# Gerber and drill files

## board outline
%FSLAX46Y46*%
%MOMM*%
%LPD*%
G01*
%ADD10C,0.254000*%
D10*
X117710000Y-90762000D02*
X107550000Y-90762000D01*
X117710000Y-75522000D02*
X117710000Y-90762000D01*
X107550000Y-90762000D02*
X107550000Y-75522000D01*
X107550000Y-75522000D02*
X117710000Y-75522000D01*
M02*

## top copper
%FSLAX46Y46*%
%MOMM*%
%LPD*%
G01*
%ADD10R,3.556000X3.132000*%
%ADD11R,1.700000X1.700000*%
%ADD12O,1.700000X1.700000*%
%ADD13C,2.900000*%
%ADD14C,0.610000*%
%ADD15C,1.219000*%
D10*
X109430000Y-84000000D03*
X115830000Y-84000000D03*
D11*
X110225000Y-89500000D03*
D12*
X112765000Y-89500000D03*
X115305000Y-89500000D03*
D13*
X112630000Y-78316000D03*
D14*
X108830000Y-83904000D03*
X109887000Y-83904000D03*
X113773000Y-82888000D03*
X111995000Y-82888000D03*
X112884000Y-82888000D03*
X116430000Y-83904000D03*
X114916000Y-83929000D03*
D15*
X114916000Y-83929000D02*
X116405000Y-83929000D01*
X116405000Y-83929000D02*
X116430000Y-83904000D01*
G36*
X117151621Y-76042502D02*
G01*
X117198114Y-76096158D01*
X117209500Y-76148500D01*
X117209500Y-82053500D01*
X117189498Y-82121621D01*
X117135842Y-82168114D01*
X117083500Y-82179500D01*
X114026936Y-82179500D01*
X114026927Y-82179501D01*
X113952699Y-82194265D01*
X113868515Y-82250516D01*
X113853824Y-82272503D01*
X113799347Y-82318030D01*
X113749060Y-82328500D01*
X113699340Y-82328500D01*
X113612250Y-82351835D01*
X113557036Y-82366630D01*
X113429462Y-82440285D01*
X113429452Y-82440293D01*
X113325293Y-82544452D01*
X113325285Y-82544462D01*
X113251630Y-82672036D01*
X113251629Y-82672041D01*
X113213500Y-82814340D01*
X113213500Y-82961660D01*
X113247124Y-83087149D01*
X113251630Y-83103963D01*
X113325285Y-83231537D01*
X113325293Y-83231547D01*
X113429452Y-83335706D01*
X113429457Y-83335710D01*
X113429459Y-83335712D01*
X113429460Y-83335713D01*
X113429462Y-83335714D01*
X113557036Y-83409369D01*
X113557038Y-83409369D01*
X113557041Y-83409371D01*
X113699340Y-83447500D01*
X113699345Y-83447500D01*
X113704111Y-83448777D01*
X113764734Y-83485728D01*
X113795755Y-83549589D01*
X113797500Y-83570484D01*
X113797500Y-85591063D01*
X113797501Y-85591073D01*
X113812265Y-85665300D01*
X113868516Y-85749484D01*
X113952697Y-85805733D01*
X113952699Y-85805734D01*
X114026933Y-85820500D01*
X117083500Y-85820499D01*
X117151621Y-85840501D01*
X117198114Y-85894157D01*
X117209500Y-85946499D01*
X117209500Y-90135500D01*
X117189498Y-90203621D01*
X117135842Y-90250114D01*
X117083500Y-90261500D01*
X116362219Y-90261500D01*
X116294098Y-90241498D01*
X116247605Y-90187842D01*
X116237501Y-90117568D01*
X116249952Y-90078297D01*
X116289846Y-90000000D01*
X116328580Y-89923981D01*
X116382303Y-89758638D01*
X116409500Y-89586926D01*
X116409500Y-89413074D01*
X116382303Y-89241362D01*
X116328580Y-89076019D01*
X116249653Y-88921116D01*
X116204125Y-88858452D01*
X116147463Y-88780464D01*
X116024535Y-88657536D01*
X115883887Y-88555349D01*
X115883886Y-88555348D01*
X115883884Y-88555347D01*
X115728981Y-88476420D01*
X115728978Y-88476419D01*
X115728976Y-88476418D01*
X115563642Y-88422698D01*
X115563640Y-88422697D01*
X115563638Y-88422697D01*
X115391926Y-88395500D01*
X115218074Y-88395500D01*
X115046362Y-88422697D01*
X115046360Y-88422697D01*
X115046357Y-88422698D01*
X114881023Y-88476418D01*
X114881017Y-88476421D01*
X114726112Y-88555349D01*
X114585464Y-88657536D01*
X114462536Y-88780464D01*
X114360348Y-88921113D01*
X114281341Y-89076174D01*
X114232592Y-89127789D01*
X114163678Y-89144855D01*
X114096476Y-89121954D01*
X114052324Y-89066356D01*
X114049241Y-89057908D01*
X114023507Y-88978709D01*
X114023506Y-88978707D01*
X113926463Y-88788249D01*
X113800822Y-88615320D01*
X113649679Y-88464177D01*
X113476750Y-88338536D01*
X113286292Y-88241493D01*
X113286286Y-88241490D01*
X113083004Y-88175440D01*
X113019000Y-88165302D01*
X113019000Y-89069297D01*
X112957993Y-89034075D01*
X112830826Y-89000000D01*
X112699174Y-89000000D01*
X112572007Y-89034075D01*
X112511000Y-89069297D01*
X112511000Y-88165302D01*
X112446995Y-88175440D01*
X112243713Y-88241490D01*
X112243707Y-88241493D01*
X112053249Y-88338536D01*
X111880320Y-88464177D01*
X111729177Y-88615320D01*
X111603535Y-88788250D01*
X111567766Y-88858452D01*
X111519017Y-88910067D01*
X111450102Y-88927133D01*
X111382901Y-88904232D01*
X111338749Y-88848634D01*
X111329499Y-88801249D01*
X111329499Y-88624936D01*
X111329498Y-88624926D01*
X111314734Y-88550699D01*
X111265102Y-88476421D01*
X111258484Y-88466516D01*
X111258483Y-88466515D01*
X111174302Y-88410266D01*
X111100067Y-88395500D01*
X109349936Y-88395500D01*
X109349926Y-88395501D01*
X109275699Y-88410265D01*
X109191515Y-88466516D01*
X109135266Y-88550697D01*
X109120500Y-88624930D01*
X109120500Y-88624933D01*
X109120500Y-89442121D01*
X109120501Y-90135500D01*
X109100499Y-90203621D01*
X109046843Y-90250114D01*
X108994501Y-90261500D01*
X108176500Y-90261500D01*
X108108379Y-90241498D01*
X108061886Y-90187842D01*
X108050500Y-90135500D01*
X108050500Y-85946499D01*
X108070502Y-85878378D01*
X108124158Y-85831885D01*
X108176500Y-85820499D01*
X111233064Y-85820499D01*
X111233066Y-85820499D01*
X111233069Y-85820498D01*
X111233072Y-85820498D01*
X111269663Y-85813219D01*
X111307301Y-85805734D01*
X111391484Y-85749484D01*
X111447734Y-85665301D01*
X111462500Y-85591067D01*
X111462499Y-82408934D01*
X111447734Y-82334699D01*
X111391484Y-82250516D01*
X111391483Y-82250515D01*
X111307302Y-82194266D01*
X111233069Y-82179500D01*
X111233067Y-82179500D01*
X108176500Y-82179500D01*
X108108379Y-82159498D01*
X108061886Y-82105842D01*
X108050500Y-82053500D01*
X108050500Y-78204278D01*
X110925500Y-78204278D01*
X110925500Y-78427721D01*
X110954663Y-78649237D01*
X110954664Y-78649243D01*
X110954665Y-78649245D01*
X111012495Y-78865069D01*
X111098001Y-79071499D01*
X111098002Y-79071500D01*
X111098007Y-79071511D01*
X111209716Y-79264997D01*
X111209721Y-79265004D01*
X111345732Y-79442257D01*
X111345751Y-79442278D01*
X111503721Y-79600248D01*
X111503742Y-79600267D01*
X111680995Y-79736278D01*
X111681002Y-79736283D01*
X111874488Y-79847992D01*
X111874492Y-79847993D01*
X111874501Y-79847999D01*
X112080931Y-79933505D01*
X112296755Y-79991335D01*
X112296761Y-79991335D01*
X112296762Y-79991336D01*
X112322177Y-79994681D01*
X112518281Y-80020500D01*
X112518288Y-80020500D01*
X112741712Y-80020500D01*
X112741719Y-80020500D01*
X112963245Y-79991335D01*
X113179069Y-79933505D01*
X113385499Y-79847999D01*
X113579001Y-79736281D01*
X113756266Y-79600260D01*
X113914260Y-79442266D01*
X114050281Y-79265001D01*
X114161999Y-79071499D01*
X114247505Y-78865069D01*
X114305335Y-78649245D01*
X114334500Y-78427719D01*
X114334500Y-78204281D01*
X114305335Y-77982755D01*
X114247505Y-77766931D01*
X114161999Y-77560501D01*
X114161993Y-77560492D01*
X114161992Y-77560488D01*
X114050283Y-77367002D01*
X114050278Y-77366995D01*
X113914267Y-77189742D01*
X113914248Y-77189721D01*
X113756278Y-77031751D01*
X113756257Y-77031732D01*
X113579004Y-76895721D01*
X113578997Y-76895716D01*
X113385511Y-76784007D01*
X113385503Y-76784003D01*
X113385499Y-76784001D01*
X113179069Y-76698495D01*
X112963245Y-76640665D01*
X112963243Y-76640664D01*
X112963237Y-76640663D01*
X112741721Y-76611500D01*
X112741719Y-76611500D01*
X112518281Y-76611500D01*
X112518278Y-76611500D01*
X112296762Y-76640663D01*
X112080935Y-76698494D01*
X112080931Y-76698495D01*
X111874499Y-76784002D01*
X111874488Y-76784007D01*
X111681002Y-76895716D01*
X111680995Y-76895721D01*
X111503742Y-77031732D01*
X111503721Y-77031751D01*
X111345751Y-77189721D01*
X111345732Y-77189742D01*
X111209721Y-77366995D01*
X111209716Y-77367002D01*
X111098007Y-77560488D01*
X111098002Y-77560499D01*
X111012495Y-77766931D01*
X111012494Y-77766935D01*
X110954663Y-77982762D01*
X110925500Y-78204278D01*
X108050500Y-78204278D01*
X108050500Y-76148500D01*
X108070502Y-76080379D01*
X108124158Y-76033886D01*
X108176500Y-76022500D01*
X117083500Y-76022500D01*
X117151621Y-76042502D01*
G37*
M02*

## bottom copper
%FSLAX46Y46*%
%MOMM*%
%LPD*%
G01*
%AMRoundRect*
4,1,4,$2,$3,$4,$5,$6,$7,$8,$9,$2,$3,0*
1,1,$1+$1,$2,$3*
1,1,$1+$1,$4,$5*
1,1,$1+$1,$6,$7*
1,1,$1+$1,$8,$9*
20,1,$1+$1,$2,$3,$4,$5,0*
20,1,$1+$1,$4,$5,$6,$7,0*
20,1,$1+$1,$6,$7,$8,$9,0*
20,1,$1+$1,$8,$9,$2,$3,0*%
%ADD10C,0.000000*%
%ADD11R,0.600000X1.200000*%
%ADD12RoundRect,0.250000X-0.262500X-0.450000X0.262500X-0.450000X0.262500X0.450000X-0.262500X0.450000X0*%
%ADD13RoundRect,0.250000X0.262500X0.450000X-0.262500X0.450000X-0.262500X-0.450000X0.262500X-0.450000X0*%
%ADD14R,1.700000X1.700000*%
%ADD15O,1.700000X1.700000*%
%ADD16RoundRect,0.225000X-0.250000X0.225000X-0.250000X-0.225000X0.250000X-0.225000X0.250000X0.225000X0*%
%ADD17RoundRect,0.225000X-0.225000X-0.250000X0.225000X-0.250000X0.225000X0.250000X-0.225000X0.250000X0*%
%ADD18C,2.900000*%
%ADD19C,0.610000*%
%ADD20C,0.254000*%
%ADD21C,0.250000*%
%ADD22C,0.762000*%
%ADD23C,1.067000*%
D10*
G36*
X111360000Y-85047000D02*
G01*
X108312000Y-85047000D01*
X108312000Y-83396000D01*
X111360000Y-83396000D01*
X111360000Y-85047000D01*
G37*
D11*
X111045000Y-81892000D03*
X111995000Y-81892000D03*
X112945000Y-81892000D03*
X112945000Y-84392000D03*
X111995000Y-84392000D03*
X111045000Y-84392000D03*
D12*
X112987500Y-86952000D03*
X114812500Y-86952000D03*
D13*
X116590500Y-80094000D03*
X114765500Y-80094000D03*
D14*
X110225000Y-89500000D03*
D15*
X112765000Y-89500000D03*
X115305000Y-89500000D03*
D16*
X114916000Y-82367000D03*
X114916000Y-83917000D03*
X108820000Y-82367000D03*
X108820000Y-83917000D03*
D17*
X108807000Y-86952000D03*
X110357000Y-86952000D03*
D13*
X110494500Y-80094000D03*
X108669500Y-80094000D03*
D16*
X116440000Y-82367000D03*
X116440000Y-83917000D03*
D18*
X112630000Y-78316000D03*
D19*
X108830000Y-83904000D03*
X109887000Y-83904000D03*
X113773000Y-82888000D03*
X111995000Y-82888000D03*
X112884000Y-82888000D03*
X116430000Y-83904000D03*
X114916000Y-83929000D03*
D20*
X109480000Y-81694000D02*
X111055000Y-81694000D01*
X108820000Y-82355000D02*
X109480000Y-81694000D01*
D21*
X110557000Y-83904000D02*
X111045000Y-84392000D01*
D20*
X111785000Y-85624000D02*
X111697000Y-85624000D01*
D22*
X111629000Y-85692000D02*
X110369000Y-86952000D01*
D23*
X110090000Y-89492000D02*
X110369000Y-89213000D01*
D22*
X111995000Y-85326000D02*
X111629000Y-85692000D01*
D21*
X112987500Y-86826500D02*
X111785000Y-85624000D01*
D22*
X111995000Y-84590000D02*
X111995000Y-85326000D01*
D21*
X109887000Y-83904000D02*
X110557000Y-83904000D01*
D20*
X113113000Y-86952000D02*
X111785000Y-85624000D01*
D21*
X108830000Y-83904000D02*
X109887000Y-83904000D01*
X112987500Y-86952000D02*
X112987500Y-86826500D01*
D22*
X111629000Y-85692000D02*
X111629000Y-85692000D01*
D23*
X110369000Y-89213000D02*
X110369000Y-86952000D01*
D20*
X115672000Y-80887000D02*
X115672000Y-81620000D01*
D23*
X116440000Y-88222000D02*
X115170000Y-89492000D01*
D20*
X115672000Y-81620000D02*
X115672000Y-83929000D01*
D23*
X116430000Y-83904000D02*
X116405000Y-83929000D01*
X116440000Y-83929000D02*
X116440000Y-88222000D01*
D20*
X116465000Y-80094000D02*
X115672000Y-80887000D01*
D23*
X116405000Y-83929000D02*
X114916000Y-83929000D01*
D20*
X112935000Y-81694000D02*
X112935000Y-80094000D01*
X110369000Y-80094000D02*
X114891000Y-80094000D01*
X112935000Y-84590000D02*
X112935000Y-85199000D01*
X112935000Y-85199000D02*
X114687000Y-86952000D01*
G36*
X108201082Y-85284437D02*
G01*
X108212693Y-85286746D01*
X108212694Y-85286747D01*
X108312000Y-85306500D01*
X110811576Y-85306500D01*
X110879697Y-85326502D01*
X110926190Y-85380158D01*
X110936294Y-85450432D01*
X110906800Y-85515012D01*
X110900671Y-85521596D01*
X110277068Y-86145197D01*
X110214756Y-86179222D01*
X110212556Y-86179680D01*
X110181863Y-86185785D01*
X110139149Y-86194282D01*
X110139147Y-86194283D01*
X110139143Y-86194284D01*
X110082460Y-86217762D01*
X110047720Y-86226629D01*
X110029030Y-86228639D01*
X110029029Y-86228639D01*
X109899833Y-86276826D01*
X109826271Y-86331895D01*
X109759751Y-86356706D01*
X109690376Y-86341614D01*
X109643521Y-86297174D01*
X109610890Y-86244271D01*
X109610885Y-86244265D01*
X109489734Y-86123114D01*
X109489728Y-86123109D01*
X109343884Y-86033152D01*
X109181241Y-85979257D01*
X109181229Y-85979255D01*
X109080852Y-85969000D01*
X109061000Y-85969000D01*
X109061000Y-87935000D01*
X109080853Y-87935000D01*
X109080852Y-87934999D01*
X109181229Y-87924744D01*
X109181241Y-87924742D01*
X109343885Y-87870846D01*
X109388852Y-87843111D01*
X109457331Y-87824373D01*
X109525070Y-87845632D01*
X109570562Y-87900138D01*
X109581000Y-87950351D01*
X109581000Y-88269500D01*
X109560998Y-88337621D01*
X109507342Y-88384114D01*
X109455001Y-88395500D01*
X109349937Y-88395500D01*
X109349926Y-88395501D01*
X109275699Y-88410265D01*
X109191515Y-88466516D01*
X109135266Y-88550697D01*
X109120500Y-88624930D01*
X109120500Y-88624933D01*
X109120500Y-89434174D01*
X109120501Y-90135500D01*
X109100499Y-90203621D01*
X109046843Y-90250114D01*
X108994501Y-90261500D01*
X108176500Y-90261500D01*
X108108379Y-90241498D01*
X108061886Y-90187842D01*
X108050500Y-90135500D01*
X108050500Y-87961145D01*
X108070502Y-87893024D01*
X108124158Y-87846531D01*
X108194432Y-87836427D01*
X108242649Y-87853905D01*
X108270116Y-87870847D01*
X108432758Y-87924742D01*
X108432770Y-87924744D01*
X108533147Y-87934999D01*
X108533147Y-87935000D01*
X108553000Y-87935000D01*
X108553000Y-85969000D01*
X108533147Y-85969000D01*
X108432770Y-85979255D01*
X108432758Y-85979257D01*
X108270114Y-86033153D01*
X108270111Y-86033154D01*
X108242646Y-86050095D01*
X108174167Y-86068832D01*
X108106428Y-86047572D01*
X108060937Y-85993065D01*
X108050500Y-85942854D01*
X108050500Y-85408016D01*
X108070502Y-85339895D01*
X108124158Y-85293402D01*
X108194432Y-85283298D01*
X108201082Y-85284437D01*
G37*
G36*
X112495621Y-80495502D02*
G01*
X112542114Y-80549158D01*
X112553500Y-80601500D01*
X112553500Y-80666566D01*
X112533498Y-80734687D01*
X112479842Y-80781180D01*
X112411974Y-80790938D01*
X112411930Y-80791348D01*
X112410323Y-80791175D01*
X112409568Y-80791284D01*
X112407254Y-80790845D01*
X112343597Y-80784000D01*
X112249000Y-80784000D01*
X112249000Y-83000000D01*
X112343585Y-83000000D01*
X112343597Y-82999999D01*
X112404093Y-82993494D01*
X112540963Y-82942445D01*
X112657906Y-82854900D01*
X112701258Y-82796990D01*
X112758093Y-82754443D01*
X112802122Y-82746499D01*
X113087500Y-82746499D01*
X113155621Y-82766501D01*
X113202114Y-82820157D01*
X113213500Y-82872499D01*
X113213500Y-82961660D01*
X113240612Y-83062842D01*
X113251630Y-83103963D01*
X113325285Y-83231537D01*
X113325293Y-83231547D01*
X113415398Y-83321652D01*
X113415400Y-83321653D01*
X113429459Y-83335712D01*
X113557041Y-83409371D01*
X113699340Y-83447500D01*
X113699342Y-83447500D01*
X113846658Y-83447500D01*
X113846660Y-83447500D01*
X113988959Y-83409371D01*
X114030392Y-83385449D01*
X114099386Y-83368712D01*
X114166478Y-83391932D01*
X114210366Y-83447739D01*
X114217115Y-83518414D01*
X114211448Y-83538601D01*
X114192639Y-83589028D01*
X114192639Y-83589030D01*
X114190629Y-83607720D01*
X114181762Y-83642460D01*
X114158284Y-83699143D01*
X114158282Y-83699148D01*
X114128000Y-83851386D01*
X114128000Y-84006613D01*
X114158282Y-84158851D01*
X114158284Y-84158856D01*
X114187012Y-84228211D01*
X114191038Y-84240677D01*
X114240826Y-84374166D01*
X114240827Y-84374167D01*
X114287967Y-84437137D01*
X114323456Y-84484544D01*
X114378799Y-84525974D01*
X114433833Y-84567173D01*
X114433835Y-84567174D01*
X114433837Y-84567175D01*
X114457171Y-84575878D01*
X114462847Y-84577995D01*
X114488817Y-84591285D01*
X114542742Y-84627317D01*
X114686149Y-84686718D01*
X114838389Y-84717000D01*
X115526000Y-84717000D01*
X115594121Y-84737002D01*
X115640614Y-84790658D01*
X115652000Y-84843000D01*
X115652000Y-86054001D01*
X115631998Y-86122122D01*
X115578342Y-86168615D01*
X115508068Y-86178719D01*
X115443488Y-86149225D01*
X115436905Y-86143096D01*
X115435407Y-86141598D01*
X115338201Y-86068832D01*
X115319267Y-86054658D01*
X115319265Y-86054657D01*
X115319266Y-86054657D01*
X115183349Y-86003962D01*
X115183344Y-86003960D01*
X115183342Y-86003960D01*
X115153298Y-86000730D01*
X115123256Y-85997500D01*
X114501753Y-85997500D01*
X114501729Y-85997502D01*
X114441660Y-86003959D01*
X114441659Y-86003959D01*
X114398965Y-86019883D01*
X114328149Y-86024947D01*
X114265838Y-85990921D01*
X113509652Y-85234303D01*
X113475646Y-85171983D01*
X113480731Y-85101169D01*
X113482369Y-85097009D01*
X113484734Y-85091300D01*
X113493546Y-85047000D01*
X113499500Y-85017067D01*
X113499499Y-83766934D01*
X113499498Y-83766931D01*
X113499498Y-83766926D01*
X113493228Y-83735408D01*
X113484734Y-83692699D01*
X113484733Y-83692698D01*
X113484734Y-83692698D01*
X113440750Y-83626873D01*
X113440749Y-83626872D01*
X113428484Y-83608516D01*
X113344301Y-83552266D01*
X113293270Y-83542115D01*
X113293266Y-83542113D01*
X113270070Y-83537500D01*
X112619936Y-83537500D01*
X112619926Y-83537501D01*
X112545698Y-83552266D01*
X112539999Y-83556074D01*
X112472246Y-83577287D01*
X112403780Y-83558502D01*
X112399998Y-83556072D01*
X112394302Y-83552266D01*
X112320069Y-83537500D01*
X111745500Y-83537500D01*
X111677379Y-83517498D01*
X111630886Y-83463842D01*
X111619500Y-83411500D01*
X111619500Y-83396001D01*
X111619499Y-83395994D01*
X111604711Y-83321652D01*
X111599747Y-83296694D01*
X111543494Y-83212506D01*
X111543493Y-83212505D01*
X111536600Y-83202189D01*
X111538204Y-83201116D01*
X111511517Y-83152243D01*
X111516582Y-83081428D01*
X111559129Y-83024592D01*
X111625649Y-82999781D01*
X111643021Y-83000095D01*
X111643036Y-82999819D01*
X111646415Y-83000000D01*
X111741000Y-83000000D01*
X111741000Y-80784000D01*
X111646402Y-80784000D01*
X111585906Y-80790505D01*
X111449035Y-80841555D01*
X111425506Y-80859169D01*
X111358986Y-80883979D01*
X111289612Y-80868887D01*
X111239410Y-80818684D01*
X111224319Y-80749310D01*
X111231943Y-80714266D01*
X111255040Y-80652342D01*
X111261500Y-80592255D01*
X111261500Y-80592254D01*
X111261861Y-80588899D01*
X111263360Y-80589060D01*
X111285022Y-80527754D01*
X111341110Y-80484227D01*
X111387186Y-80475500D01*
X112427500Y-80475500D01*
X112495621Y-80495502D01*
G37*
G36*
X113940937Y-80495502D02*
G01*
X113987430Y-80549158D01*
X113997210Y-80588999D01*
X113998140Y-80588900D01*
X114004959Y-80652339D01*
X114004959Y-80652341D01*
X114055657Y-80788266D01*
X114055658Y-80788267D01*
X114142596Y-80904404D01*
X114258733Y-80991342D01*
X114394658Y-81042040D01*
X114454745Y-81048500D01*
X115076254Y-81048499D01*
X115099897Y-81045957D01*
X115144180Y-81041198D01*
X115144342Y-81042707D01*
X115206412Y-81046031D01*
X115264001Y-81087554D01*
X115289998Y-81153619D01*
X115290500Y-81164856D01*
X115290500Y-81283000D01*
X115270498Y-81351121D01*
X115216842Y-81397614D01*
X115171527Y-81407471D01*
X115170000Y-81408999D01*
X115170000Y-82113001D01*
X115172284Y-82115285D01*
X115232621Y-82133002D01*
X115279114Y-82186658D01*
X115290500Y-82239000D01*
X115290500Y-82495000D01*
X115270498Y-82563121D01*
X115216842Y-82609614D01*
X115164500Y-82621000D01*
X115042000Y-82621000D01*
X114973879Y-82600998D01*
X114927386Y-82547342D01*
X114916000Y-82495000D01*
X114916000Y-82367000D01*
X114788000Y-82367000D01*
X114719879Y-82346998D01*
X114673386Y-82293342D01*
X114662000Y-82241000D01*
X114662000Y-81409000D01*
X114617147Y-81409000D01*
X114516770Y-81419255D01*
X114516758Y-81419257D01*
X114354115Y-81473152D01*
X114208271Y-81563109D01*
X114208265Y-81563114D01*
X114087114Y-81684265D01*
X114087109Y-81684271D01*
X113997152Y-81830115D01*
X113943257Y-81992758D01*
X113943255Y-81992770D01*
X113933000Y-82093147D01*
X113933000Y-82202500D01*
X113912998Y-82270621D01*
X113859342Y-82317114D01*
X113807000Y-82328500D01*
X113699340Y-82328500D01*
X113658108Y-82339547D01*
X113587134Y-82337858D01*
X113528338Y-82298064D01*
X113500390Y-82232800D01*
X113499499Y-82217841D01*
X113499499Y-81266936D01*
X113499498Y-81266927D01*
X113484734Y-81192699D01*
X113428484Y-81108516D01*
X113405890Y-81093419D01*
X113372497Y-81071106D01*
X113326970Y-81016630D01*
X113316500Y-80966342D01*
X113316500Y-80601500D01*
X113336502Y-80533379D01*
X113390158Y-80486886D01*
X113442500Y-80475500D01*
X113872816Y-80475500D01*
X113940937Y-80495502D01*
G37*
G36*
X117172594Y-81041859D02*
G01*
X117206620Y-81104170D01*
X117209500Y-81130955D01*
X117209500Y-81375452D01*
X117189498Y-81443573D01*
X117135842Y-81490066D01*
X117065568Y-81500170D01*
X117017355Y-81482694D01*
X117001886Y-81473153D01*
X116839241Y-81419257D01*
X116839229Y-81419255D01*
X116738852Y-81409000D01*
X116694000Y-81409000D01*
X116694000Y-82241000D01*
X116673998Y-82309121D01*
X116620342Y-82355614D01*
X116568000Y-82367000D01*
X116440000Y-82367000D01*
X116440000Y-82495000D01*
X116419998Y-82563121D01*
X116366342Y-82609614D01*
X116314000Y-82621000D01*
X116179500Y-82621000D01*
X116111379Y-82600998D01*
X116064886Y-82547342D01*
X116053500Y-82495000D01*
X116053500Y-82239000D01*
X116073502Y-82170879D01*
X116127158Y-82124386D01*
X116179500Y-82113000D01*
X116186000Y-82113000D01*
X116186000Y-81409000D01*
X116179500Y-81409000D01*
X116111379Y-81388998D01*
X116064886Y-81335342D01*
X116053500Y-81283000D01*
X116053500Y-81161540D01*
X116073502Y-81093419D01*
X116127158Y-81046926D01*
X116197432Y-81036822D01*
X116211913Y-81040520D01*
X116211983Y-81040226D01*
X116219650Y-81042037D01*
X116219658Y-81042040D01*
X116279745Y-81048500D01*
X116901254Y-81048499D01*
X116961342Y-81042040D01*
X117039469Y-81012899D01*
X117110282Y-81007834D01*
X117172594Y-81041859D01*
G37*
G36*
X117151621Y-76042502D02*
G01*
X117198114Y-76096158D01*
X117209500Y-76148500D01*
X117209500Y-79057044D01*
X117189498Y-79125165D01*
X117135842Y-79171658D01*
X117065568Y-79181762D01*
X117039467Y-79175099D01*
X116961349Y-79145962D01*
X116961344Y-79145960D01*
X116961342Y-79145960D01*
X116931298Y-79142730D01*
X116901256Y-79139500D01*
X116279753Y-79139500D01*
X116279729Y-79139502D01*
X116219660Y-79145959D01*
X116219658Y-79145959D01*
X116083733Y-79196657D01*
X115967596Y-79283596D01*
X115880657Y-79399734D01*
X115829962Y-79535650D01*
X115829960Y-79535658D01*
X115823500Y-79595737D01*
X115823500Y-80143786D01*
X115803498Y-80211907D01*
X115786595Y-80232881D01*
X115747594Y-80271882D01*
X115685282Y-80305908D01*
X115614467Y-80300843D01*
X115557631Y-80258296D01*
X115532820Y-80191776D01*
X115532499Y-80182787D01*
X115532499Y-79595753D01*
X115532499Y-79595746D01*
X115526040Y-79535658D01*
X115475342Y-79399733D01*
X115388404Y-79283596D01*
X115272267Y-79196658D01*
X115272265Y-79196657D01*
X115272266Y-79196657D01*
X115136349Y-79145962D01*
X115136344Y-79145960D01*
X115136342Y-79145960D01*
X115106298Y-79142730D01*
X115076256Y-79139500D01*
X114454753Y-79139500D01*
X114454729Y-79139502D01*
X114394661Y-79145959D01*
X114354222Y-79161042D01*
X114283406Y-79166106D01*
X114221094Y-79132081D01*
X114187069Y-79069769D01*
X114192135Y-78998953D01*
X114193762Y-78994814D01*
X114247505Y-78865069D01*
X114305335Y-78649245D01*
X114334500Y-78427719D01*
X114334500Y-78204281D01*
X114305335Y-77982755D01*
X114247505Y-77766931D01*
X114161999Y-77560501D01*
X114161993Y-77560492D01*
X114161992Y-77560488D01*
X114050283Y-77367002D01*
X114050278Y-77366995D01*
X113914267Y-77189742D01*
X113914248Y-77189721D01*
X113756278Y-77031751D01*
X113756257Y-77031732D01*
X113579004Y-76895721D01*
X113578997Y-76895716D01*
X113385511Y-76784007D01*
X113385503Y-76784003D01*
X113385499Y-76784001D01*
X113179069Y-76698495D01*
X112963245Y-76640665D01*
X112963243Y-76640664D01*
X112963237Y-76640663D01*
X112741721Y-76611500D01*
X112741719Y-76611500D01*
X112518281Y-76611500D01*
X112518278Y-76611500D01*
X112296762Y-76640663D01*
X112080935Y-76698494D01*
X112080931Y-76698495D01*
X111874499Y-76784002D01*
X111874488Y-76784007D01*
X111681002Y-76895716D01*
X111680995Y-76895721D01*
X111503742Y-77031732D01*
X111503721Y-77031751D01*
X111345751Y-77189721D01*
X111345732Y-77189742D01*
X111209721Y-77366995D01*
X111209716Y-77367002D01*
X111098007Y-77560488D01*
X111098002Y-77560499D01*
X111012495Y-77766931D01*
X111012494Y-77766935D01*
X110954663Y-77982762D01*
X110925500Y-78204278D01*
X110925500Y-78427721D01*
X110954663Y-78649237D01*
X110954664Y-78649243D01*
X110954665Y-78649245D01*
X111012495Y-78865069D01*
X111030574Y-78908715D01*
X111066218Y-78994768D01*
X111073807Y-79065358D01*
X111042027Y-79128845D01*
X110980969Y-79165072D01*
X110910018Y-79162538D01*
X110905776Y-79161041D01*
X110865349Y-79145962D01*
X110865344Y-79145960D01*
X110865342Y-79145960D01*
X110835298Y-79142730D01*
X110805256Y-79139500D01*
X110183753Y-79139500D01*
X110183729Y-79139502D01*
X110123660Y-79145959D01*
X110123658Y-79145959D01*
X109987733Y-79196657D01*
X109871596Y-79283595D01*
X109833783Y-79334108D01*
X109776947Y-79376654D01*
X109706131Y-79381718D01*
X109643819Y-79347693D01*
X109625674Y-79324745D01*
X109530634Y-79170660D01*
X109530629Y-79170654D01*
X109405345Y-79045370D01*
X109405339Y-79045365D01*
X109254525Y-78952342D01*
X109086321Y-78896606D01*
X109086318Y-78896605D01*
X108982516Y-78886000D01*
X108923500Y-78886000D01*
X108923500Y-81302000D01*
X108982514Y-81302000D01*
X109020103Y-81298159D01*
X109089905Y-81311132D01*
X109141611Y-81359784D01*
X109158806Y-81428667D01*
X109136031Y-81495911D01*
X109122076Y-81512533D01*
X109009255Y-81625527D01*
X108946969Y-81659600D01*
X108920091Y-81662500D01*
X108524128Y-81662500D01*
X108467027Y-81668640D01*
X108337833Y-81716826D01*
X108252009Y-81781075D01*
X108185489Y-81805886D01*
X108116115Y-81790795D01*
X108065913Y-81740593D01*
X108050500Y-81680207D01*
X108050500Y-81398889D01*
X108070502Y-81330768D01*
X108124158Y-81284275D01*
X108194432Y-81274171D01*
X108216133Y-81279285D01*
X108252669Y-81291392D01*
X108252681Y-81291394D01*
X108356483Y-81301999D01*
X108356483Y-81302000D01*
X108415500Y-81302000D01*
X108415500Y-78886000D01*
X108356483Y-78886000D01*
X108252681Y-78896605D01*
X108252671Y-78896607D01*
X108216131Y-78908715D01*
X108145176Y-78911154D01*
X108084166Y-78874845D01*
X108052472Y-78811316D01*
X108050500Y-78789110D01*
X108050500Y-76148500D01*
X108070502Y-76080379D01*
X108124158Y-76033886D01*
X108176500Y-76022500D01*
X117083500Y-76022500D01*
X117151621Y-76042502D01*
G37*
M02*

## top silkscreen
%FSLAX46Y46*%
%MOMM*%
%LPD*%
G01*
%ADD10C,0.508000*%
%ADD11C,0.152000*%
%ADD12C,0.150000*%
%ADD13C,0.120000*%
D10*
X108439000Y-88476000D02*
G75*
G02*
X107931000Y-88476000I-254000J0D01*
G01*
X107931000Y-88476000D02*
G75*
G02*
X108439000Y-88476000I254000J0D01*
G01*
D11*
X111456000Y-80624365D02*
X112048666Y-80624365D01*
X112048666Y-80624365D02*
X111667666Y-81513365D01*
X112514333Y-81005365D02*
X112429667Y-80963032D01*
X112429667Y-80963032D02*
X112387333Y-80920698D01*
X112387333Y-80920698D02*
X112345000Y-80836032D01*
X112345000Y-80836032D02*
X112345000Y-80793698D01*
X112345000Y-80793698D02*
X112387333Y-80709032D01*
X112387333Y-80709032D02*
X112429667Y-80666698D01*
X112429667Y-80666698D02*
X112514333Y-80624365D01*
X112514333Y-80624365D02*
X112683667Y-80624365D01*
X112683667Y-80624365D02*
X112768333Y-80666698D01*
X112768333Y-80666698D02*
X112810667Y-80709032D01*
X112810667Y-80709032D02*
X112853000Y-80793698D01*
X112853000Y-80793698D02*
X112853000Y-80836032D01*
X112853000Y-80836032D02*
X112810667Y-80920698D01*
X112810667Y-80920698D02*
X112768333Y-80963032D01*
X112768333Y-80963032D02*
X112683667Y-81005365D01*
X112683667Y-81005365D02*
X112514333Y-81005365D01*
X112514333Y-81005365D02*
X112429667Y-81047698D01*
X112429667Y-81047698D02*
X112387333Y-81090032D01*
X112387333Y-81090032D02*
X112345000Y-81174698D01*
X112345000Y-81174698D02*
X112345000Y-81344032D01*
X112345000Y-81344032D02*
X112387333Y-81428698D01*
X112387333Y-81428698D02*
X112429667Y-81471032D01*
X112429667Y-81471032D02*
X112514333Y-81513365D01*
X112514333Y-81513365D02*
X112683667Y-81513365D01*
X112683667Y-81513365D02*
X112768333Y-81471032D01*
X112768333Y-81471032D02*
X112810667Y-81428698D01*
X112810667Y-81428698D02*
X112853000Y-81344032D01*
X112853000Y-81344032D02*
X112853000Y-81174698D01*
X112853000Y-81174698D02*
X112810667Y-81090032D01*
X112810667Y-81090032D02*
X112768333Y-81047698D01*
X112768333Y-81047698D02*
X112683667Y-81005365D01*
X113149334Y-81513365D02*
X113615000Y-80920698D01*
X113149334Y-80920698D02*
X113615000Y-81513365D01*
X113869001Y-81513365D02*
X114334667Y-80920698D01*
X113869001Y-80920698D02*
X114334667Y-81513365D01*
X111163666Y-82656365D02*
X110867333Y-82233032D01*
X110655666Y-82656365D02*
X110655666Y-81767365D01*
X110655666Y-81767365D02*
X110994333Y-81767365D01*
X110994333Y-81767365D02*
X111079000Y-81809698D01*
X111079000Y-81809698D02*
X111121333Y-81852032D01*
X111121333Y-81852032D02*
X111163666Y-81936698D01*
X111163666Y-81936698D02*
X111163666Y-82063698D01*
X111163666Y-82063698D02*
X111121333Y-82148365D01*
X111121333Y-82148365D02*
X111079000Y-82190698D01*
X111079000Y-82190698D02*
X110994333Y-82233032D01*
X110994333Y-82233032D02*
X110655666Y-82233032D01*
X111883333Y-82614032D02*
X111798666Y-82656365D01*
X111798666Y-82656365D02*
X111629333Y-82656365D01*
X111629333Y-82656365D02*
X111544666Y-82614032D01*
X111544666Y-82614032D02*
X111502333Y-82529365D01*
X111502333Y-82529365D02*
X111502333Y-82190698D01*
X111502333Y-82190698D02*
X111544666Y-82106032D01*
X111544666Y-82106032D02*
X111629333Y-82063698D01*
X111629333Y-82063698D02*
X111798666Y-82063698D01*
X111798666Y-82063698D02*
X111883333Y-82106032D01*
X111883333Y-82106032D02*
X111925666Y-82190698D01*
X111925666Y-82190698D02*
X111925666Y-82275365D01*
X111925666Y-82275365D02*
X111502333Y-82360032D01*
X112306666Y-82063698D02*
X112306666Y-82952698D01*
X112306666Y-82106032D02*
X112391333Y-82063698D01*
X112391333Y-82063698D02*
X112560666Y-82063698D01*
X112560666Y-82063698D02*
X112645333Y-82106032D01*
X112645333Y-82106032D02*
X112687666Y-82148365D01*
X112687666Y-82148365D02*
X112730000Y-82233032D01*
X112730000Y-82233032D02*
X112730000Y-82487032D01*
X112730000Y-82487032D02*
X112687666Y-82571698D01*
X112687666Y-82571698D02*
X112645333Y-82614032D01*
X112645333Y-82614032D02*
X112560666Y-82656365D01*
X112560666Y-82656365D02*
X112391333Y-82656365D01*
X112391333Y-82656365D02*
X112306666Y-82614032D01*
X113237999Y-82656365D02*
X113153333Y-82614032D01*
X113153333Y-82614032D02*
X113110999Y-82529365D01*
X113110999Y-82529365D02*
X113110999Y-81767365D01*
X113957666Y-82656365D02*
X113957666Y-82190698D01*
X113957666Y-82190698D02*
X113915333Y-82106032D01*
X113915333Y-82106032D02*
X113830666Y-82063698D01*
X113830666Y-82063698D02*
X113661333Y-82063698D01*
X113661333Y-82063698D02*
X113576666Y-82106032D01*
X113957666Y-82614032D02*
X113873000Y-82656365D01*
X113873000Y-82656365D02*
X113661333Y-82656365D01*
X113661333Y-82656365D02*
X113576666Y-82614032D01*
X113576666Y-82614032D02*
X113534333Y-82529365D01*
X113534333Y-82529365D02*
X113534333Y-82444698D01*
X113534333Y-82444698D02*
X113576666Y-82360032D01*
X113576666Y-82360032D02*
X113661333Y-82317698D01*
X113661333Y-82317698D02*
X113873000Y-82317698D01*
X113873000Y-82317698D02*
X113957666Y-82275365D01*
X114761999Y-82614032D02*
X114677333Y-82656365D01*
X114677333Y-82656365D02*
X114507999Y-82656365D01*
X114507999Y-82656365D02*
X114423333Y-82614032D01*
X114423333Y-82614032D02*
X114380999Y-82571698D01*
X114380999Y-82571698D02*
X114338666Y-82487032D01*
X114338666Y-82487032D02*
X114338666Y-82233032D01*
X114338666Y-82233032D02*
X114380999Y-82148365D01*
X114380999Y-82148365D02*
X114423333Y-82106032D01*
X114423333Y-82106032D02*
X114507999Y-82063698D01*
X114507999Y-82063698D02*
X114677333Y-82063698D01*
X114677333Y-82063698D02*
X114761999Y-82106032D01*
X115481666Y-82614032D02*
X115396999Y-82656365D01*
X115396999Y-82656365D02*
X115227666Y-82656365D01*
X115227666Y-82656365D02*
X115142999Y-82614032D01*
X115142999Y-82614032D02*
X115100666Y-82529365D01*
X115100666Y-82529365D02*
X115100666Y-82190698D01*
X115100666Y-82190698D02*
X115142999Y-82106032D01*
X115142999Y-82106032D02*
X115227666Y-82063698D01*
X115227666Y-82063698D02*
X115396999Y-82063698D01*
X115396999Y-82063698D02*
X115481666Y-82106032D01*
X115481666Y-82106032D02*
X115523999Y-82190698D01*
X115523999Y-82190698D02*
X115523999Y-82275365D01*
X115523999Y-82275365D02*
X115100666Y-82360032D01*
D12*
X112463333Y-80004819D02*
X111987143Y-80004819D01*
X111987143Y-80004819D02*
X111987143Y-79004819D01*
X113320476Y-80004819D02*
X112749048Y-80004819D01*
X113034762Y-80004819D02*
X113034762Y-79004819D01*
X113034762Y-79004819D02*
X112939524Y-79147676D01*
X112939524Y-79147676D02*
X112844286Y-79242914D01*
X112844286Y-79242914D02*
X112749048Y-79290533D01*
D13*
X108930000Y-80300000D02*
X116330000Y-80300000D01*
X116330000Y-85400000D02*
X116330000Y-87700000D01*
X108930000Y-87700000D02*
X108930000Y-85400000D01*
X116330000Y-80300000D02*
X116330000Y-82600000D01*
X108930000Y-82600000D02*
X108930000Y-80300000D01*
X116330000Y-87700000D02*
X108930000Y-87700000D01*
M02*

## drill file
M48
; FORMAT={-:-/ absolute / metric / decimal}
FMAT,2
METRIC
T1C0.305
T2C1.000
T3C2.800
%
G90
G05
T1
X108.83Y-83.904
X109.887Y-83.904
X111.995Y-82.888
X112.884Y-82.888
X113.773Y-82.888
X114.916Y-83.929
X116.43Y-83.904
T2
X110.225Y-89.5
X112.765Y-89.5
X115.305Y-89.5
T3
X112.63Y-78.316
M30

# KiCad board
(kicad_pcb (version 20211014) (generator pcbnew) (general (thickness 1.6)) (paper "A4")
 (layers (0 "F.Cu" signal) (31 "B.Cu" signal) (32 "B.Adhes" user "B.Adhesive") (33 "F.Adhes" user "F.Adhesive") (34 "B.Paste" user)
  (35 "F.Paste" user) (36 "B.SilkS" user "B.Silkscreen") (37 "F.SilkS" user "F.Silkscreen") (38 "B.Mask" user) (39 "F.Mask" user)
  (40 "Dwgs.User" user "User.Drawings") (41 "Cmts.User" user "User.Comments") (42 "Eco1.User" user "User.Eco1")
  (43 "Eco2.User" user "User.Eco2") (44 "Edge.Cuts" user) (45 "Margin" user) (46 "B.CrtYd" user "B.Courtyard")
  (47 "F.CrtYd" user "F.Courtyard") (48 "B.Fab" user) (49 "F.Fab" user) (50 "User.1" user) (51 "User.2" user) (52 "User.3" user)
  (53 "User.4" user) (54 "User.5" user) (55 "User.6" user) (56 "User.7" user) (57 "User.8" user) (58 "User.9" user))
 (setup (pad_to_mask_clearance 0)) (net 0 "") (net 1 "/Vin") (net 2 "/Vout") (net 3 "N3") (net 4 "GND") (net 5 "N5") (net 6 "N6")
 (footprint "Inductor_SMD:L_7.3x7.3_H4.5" (layer "F.Cu") (at 112.63 84)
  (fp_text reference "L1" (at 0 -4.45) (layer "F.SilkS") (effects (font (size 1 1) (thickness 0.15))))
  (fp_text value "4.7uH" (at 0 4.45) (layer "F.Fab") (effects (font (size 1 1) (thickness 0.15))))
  (fp_line (start -3.7 -3.7) (end 3.7 -3.7) (layer "F.SilkS") (width 0.12))
  (fp_line (start 3.7 1.4) (end 3.7 3.7) (layer "F.SilkS") (width 0.12))
  (fp_line (start -3.7 3.7) (end -3.7 1.4) (layer "F.SilkS") (width 0.12))
  (fp_line (start 3.7 -3.7) (end 3.7 -1.4) (layer "F.SilkS") (width 0.12))
  (fp_line (start -3.7 -1.4) (end -3.7 -3.7) (layer "F.SilkS") (width 0.12))
  (fp_line (start 3.7 3.7) (end -3.7 3.7) (layer "F.SilkS") (width 0.12))
  (pad "1" smd rect (at -3.2 0) (size 3.556 3.132) (layers "F.Cu" "F.Paste" "F.Mask") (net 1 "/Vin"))
  (pad "2" smd rect (at 3.2 0) (size 3.556 3.132) (layers "F.Cu" "F.Paste" "F.Mask") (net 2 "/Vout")))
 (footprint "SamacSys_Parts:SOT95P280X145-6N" (layer "B.Cu") (at 111.995 83.142 -90)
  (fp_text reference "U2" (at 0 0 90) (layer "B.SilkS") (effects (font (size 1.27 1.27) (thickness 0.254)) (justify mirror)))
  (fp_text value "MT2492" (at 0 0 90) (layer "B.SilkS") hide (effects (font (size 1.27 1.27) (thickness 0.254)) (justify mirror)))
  (pad "1" smd rect locked (at -1.25 0.95 180) (size 0.6 1.2) (layers "B.Cu" "B.Paste" "B.Mask") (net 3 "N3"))
  (pad "2" smd rect locked (at -1.25 0 180) (size 0.6 1.2) (layers "B.Cu" "B.Paste" "B.Mask") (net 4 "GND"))
  (pad "3" smd rect locked (at -1.25 -0.95 180) (size 0.6 1.2) (layers "B.Cu" "B.Paste" "B.Mask") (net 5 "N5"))
  (pad "4" smd rect locked (at 1.25 -0.95 180) (size 0.6 1.2) (layers "B.Cu" "B.Paste" "B.Mask") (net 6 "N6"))
  (pad "5" smd rect locked (at 1.25 0 180) (size 0.6 1.2) (layers "B.Cu" "B.Paste" "B.Mask") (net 1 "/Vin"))
  (pad "6" smd rect locked (at 1.25 0.95 180) (size 0.6 1.2) (layers "B.Cu" "B.Paste" "B.Mask") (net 1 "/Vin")))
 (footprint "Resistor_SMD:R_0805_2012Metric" (layer "B.Cu") (at 113.9 86.952)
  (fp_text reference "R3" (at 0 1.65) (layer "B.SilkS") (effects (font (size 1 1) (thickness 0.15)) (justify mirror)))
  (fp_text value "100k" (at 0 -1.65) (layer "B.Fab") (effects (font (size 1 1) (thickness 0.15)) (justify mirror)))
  (pad "1" smd roundrect locked (at -0.9125 0) (size 1.025 1.4) (layers "B.Cu" "B.Paste" "B.Mask") (roundrect_rratio 0.243902)
   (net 1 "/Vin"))
  (pad "2" smd roundrect locked (at 0.9125 0) (size 1.025 1.4) (layers "B.Cu" "B.Paste" "B.Mask") (roundrect_rratio 0.243902) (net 6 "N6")))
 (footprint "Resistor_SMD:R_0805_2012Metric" (layer "B.Cu") (at 115.678 80.094 180)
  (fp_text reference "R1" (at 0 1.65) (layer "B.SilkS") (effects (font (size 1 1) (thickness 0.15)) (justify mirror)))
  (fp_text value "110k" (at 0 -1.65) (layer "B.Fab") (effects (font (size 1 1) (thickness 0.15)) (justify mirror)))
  (pad "1" smd roundrect locked (at -0.9125 0 180) (size 1.025 1.4) (layers "B.Cu" "B.Paste" "B.Mask") (roundrect_rratio 0.243902)
   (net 2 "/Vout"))
  (pad "2" smd roundrect locked (at 0.9125 0 180) (size 1.025 1.4) (layers "B.Cu" "B.Paste" "B.Mask") (roundrect_rratio 0.243902)
   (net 5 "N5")))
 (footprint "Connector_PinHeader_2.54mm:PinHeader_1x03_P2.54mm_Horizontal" (layer "B.Cu") (at 110.225 89.5 -90)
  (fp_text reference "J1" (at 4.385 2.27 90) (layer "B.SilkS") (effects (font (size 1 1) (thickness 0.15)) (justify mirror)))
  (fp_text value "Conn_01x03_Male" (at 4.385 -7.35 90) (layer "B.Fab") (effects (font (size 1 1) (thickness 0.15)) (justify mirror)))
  (pad "1" thru_hole rect locked (at 0 0 270) (size 1.7 1.7) (drill 1) (layers *.Cu *.Mask) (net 1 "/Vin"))
  (pad "2" thru_hole oval locked (at 0 -2.54 270) (size 1.7 1.7) (drill 1) (layers *.Cu *.Mask) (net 4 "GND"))
  (pad "3" thru_hole oval locked (at 0 -5.08 270) (size 1.7 1.7) (drill 1) (layers *.Cu *.Mask) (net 2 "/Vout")))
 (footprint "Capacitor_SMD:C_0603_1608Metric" (layer "B.Cu") (at 114.916 83.142 -90)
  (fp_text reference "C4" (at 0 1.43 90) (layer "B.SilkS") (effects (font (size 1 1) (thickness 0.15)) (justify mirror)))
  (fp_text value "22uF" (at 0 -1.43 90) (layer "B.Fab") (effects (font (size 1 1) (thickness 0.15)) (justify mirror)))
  (pad "1" smd roundrect locked (at -0.775 0 270) (size 0.9 0.95) (layers "B.Cu" "B.Paste" "B.Mask") (roundrect_rratio 0.25) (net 4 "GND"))
  (pad "2" smd roundrect locked (at 0.775 0 270) (size 0.9 0.95) (layers "B.Cu" "B.Paste" "B.Mask") (roundrect_rratio 0.25) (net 2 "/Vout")))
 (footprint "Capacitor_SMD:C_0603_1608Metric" (layer "B.Cu") (at 108.82 83.142 -90)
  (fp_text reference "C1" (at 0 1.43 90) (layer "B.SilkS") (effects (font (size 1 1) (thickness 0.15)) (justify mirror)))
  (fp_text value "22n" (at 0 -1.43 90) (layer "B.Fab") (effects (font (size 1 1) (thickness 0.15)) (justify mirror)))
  (pad "1" smd roundrect locked (at -0.775 0 270) (size 0.9 0.95) (layers "B.Cu" "B.Paste" "B.Mask") (roundrect_rratio 0.25) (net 3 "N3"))
  (pad "2" smd roundrect locked (at 0.775 0 270) (size 0.9 0.95) (layers "B.Cu" "B.Paste" "B.Mask") (roundrect_rratio 0.25) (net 1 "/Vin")))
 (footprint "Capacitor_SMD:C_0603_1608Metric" (layer "B.Cu") (at 109.582 86.952)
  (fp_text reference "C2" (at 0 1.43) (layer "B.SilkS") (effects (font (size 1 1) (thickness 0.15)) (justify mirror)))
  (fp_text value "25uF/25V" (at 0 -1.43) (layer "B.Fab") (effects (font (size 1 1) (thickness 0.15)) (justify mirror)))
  (pad "1" smd roundrect locked (at -0.775 0) (size 0.9 0.95) (layers "B.Cu" "B.Paste" "B.Mask") (roundrect_rratio 0.25) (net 4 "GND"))
  (pad "2" smd roundrect locked (at 0.775 0) (size 0.9 0.95) (layers "B.Cu" "B.Paste" "B.Mask") (roundrect_rratio 0.25) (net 1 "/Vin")))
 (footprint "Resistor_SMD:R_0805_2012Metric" (layer "B.Cu") (at 109.582 80.094 180)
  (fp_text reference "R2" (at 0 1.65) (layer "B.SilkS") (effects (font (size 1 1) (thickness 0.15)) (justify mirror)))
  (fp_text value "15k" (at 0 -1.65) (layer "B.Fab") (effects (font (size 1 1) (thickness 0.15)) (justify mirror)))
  (pad "1" smd roundrect locked (at -0.9125 0 180) (size 1.025 1.4) (layers "B.Cu" "B.Paste" "B.Mask") (roundrect_rratio 0.243902)
   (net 5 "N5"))
  (pad "2" smd roundrect locked (at 0.9125 0 180) (size 1.025 1.4) (layers "B.Cu" "B.Paste" "B.Mask") (roundrect_rratio 0.243902)
   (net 4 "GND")))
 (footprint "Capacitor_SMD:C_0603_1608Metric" (layer "B.Cu") (at 116.44 83.142 -90)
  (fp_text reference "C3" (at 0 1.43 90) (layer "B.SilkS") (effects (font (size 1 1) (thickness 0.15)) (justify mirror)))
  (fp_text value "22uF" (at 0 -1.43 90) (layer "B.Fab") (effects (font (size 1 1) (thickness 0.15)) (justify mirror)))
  (pad "1" smd roundrect locked (at -0.775 0 270) (size 0.9 0.95) (layers "B.Cu" "B.Paste" "B.Mask") (roundrect_rratio 0.25) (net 4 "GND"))
  (pad "2" smd roundrect locked (at 0.775 0 270) (size 0.9 0.95) (layers "B.Cu" "B.Paste" "B.Mask") (roundrect_rratio 0.25) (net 2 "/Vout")))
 (gr_poly (pts (xy 108.312 83.396) (xy 111.36 83.396) (xy 111.36 85.047) (xy 108.312 85.047)) (layer "B.Cu") (width 0) (fill solid))
 (gr_circle (center 108.185 88.476) (end 108.439 88.476) (layer "F.SilkS") (width 0.508) (fill none))
 (gr_line (start 117.71 90.762) (end 107.55 90.762) (layer "Edge.Cuts") (width 0.254))
 (gr_line (start 117.71 75.522) (end 117.71 90.762) (layer "Edge.Cuts") (width 0.254))
 (gr_line (start 107.55 90.762) (end 107.55 75.522) (layer "Edge.Cuts") (width 0.254))
 (gr_line (start 107.55 75.522) (end 117.71 75.522) (layer "Edge.Cuts") (width 0.254))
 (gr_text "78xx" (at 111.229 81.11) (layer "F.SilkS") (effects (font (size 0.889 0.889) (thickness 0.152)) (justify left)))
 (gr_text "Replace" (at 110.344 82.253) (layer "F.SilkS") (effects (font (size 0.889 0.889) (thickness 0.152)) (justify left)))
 (via (at 112.63 78.316) (size 2.9) (drill 2.8) (layers "F.Cu" "B.Cu") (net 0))
 (segment (start 109.48 81.694) (end 111.055 81.694) (width 0.254) (layer "B.Cu") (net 3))
 (segment (start 108.82 82.355) (end 109.48 81.694) (width 0.254) (layer "B.Cu") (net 3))
 (via (at 108.83 83.904) (size 0.61) (drill 0.305) (layers "F.Cu" "B.Cu") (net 1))
 (via (at 109.887 83.904) (size 0.61) (drill 0.305) (layers "F.Cu" "B.Cu") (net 1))
 (segment (start 110.557 83.904) (end 111.045 84.392) (width 0.25) (layer "B.Cu") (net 1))
 (segment (start 111.785 85.624) (end 111.697 85.624) (width 0.254) (layer "B.Cu") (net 1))
 (segment (start 111.629 85.692) (end 110.369 86.952) (width 0.762) (layer "B.Cu") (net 1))
 (segment (start 110.09 89.492) (end 110.369 89.213) (width 1.067) (layer "B.Cu") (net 1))
 (segment (start 111.995 85.326) (end 111.629 85.692) (width 0.762) (layer "B.Cu") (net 1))
 (segment (start 112.9875 86.8265) (end 111.785 85.624) (width 0.25) (layer "B.Cu") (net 1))
 (segment (start 111.995 84.59) (end 111.995 85.326) (width 0.762) (layer "B.Cu") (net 1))
 (segment (start 109.887 83.904) (end 110.557 83.904) (width 0.25) (layer "B.Cu") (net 1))
 (segment (start 113.113 86.952) (end 111.785 85.624) (width 0.254) (layer "B.Cu") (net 1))
 (segment (start 108.83 83.904) (end 109.887 83.904) (width 0.25) (layer "B.Cu") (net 1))
 (segment (start 112.9875 86.952) (end 112.9875 86.8265) (width 0.25) (layer "B.Cu") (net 1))
 (segment (start 111.629 85.692) (end 111.629 85.692) (width 0.762) (layer "B.Cu") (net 1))
 (segment (start 110.369 89.213) (end 110.369 86.952) (width 1.067) (layer "B.Cu") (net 1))
 (via (at 113.773 82.888) (size 0.61) (drill 0.305) (layers "F.Cu" "B.Cu") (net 4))
 (via (at 111.995 82.888) (size 0.61) (drill 0.305) (layers "F.Cu" "B.Cu") (free) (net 4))
 (via (at 112.884 82.888) (size 0.61) (drill 0.305) (layers "F.Cu" "B.Cu") (free) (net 4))
 (segment (start 114.916 83.929) (end 116.405 83.929) (width 1.219) (layer "F.Cu") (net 2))
 (segment (start 116.405 83.929) (end 116.43 83.904) (width 1.219) (layer "F.Cu") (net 2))
 (via (at 116.43 83.904) (size 0.61) (drill 0.305) (layers "F.Cu" "B.Cu") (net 2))
 (via (at 114.916 83.929) (size 0.61) (drill 0.305) (layers "F.Cu" "B.Cu") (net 2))
 (segment (start 115.672 80.887) (end 115.672 81.62) (width 0.254) (layer "B.Cu") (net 2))
 (segment (start 116.44 88.222) (end 115.17 89.492) (width 1.067) (layer "B.Cu") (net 2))
 (segment (start 115.672 81.62) (end 115.672 83.929) (width 0.254) (layer "B.Cu") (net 2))
 (segment (start 116.43 83.904) (end 116.405 83.929) (width 1.067) (layer "B.Cu") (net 2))
 (segment (start 116.44 83.929) (end 116.44 88.222) (width 1.067) (layer "B.Cu") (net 2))
 (segment (start 116.465 80.094) (end 115.672 80.887) (width 0.254) (layer "B.Cu") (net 2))
 (segment (start 116.405 83.929) (end 114.916 83.929) (width 1.067) (layer "B.Cu") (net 2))
 (segment (start 112.935 81.694) (end 112.935 80.094) (width 0.254) (layer "B.Cu") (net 5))
 (segment (start 110.369 80.094) (end 114.891 80.094) (width 0.254) (layer "B.Cu") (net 5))
 (segment (start 112.935 84.59) (end 112.935 85.199) (width 0.254) (layer "B.Cu") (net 6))
 (segment (start 112.935 85.199) (end 114.687 86.952) (width 0.254) (layer "B.Cu") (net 6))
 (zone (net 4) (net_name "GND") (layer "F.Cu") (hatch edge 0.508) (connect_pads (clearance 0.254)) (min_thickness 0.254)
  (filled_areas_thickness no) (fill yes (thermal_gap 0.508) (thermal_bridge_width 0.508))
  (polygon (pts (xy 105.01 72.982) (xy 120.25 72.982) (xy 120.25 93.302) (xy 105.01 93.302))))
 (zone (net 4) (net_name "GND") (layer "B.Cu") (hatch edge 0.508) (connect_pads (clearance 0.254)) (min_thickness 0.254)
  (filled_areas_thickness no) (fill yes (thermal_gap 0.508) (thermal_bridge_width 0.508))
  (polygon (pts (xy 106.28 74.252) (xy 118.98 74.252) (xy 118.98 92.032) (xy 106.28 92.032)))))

